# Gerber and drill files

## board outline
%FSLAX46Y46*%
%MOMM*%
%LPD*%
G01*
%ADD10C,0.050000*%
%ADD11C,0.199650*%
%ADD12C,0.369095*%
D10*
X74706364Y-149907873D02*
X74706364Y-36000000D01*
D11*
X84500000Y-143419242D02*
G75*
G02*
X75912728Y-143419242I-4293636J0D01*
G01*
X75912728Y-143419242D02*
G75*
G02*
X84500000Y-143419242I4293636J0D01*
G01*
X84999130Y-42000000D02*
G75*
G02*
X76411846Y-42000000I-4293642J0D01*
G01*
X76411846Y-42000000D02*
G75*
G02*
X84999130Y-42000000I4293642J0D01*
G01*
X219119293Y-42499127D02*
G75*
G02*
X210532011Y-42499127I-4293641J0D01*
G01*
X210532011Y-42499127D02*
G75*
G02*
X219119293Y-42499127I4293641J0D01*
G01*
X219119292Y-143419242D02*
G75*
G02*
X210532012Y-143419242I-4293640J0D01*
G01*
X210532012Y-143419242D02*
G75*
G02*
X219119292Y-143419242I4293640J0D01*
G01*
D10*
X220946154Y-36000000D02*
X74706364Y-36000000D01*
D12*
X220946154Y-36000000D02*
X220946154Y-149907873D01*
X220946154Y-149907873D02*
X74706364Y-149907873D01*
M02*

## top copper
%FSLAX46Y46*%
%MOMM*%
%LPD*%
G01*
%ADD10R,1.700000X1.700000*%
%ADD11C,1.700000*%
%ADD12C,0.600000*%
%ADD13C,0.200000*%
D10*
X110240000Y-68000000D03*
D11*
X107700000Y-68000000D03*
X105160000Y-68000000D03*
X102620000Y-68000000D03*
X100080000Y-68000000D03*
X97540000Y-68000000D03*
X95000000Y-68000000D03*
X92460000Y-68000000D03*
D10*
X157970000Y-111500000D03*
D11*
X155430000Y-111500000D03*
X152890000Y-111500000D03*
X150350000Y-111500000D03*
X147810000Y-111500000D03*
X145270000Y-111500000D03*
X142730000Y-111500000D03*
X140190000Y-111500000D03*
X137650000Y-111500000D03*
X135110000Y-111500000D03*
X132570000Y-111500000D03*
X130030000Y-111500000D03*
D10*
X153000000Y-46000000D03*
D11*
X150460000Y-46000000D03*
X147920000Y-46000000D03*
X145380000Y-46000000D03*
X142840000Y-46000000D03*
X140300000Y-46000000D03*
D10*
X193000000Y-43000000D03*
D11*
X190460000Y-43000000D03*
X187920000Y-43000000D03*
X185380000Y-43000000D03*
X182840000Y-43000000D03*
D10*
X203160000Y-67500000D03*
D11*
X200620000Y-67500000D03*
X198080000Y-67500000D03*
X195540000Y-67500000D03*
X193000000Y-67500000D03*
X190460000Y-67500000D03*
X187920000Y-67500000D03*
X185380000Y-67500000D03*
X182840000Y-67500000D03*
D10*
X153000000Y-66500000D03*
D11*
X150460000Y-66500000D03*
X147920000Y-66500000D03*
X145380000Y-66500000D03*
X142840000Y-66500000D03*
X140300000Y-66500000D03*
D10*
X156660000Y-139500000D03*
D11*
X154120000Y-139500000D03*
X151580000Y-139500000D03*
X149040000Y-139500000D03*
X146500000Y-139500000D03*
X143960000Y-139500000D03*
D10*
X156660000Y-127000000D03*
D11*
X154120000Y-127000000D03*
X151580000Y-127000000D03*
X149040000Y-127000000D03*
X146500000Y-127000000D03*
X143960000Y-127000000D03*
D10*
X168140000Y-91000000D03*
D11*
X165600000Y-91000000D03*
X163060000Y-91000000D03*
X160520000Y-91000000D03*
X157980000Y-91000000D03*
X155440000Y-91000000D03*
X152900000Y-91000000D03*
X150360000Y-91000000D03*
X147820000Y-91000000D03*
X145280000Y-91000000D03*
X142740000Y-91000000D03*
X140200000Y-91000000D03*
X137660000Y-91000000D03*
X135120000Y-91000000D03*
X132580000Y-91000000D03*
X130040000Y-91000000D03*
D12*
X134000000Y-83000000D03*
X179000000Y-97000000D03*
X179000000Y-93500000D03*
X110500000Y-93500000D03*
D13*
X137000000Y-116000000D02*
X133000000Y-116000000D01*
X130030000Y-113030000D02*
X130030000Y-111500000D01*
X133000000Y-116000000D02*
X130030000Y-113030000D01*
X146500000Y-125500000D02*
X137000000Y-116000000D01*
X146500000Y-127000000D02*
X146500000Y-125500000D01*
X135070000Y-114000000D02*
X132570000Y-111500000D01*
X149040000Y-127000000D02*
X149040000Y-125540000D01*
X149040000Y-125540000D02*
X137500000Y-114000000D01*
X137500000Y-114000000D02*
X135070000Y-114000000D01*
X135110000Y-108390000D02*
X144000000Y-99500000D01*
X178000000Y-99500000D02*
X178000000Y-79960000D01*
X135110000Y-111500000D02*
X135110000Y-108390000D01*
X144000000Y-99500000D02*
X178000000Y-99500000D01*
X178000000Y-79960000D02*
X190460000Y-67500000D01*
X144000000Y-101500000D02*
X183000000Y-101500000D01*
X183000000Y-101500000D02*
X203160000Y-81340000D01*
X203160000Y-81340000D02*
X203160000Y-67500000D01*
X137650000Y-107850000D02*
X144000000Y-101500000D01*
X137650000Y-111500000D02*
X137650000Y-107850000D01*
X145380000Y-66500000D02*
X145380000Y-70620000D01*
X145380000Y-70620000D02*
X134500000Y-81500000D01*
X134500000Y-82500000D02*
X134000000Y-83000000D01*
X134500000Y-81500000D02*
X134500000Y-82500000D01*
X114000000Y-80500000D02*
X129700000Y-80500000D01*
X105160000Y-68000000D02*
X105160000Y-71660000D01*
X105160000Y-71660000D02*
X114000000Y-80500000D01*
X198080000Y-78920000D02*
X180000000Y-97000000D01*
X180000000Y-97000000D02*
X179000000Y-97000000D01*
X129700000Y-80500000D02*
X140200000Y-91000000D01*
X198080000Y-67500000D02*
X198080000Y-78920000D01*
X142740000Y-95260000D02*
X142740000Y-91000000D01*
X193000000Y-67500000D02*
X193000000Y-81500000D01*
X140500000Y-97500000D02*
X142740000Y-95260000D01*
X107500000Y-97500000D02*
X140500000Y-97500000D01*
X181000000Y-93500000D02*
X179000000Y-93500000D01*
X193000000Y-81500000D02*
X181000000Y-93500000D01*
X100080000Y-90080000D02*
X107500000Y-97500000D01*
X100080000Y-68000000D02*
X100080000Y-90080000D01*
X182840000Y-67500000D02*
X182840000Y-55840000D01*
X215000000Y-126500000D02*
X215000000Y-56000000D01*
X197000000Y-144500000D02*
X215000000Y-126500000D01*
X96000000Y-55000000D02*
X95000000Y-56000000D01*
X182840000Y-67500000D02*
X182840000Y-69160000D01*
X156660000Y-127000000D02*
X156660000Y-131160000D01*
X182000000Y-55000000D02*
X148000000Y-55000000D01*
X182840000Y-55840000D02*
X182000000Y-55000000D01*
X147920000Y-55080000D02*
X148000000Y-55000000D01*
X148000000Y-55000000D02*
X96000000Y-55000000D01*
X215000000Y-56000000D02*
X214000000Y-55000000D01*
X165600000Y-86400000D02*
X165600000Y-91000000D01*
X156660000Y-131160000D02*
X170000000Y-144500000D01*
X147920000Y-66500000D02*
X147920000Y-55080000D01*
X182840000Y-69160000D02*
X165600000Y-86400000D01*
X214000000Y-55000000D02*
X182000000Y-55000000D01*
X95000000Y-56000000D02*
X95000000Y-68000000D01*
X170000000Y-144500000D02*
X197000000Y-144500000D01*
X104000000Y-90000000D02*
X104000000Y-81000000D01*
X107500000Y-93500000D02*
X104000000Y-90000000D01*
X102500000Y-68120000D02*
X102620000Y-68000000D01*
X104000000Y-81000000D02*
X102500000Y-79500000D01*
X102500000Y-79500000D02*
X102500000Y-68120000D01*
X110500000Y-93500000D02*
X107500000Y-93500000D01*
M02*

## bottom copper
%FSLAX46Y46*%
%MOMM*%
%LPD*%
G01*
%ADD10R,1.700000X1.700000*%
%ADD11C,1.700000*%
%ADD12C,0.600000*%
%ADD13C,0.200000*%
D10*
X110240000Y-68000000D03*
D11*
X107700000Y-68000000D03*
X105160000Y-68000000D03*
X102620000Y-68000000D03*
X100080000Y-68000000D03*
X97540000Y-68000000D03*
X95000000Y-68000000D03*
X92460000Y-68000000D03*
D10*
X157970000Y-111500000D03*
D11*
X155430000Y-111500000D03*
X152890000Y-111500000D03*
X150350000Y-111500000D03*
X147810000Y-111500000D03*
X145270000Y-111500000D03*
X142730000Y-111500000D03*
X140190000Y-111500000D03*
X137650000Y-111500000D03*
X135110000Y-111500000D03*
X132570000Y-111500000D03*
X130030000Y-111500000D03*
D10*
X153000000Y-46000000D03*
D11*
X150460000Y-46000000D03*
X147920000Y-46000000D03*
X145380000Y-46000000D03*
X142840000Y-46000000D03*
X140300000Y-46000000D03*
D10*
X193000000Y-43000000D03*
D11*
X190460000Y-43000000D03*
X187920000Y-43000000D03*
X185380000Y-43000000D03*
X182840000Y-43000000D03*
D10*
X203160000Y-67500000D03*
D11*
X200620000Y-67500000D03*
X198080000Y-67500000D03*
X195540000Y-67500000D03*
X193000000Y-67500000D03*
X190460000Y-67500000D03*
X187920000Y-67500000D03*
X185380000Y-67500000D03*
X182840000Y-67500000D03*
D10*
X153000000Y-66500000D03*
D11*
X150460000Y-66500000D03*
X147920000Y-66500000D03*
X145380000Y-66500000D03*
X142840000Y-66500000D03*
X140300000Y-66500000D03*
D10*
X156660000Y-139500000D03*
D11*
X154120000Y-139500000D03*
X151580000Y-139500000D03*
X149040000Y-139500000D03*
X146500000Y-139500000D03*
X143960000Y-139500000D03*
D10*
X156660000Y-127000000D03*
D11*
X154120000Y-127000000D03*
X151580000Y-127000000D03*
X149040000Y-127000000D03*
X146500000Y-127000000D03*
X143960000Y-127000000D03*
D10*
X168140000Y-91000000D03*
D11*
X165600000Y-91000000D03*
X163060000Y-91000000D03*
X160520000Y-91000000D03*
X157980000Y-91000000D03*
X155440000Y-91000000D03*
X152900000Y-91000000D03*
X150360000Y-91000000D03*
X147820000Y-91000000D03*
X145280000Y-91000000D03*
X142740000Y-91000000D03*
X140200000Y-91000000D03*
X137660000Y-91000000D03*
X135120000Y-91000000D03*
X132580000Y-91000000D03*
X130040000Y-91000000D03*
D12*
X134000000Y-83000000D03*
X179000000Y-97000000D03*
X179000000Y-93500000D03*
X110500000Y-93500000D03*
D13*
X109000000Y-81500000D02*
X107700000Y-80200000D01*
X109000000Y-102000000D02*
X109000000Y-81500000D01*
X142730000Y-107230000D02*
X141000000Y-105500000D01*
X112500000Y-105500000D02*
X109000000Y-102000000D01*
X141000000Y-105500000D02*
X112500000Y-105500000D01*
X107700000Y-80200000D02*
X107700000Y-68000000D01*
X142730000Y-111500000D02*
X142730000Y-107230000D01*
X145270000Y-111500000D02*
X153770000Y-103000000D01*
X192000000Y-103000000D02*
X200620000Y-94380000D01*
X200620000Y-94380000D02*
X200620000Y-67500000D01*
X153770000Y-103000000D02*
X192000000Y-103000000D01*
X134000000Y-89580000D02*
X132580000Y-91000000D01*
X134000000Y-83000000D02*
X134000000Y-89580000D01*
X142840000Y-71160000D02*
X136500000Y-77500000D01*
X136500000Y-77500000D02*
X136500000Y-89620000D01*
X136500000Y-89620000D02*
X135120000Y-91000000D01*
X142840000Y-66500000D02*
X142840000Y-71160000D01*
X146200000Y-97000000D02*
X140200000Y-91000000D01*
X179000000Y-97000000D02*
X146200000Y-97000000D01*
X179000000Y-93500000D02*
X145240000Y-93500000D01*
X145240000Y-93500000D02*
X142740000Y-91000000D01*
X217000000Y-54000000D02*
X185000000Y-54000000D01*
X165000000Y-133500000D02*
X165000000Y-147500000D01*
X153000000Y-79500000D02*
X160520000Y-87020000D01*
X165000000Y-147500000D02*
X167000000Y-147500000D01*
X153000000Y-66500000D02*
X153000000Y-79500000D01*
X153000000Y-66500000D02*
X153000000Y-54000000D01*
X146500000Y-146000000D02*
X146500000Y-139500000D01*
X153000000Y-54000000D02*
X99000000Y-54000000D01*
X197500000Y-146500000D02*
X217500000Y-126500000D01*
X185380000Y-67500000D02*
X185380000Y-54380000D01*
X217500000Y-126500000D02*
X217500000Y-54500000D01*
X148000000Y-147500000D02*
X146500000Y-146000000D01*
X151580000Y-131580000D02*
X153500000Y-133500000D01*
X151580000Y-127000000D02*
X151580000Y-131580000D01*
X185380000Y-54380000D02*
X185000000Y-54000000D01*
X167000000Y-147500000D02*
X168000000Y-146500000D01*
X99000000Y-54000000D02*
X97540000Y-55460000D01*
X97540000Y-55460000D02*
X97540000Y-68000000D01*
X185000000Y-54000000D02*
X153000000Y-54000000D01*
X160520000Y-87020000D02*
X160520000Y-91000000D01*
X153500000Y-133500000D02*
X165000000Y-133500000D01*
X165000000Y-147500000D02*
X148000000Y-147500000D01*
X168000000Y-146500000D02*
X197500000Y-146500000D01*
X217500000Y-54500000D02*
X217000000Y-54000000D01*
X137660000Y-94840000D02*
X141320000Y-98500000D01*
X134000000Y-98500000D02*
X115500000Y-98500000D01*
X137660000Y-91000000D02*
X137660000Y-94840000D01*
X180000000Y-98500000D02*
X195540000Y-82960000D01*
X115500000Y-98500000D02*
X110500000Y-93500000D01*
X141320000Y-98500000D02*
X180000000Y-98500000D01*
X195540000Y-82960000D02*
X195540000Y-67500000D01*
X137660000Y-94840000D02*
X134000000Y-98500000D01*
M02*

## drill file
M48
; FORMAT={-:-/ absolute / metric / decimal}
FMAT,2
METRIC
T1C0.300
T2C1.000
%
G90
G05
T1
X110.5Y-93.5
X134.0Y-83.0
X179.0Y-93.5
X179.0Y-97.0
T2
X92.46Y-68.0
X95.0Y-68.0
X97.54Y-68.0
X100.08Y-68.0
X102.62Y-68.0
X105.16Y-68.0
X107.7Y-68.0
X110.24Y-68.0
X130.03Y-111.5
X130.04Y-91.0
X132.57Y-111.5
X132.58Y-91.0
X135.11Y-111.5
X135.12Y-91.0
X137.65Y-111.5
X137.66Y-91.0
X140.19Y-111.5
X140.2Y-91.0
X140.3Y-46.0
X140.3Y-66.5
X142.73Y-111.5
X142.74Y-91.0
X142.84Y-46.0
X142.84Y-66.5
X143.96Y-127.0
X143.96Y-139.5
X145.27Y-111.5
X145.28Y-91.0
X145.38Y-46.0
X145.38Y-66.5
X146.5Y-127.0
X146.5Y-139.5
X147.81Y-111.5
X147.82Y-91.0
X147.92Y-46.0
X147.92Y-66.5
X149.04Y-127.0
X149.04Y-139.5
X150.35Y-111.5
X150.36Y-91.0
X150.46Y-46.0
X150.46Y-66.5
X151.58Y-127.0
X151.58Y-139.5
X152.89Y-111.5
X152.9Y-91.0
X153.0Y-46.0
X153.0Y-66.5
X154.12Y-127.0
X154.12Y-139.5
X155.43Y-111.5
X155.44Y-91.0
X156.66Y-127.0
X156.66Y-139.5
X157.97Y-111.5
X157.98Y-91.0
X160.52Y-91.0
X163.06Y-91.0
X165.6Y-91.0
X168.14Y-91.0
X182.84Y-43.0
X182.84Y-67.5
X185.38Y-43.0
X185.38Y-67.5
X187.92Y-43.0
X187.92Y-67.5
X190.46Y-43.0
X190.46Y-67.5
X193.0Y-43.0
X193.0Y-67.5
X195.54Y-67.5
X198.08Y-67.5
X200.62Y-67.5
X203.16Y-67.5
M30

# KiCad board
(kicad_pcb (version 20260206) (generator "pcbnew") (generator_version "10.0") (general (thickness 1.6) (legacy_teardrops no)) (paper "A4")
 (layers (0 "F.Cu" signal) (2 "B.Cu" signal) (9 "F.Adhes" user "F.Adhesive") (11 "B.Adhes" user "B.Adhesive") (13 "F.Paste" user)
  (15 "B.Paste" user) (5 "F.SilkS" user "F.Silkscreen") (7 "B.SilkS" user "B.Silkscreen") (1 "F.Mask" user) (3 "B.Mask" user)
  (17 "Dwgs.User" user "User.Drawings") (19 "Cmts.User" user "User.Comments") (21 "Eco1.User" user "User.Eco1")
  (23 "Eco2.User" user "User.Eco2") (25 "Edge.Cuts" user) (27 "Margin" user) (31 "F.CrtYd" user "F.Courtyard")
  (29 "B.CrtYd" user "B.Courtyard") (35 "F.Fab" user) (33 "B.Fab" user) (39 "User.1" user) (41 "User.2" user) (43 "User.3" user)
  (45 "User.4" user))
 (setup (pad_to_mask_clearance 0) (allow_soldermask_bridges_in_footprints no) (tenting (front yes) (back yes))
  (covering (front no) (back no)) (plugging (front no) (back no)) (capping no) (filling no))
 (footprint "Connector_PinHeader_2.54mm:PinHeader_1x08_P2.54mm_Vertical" (layer "F.Cu") (at 110.24 68 -90)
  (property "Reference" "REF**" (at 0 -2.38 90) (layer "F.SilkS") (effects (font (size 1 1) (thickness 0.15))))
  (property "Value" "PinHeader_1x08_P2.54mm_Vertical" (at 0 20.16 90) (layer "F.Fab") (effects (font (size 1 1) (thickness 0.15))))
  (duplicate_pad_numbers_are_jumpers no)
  (pad "1" thru_hole rect (at 0 0 270) (size 1.7 1.7) (drill 1) (layers "*.Cu" "*.Mask") (remove_unused_layers no))
  (pad "2" thru_hole circle (at 0 2.54 270) (size 1.7 1.7) (drill 1) (layers "*.Cu" "*.Mask") (remove_unused_layers no) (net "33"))
  (pad "3" thru_hole circle (at 0 5.08 270) (size 1.7 1.7) (drill 1) (layers "*.Cu" "*.Mask") (remove_unused_layers no) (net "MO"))
  (pad "4" thru_hole circle (at 0 7.62 270) (size 1.7 1.7) (drill 1) (layers "*.Cu" "*.Mask") (remove_unused_layers no) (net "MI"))
  (pad "5" thru_hole circle (at 0 10.16 270) (size 1.7 1.7) (drill 1) (layers "*.Cu" "*.Mask") (remove_unused_layers no) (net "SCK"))
  (pad "6" thru_hole circle (at 0 12.7 270) (size 1.7 1.7) (drill 1) (layers "*.Cu" "*.Mask") (remove_unused_layers no) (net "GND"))
  (pad "7" thru_hole circle (at 0 15.24 270) (size 1.7 1.7) (drill 1) (layers "*.Cu" "*.Mask") (remove_unused_layers no) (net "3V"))
  (pad "8" thru_hole circle (at 0 17.78 270) (size 1.7 1.7) (drill 1) (layers "*.Cu" "*.Mask") (remove_unused_layers no)))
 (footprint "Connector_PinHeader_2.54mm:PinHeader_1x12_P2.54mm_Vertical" (layer "F.Cu") (at 157.97 111.5 -90)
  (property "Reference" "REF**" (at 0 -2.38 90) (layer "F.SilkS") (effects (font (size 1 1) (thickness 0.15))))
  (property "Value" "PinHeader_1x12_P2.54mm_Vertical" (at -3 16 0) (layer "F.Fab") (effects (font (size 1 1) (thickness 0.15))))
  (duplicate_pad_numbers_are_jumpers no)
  (pad "1" thru_hole rect (at 0 0 270) (size 1.7 1.7) (drill 1) (layers "*.Cu" "*.Mask") (remove_unused_layers no))
  (pad "2" thru_hole circle (at 0 2.54 270) (size 1.7 1.7) (drill 1) (layers "*.Cu" "*.Mask") (remove_unused_layers no))
  (pad "3" thru_hole circle (at 0 5.08 270) (size 1.7 1.7) (drill 1) (layers "*.Cu" "*.Mask") (remove_unused_layers no))
  (pad "4" thru_hole circle (at 0 7.62 270) (size 1.7 1.7) (drill 1) (layers "*.Cu" "*.Mask") (remove_unused_layers no))
  (pad "5" thru_hole circle (at 0 10.16 270) (size 1.7 1.7) (drill 1) (layers "*.Cu" "*.Mask") (remove_unused_layers no))
  (pad "6" thru_hole circle (at 0 12.7 270) (size 1.7 1.7) (drill 1) (layers "*.Cu" "*.Mask") (remove_unused_layers no) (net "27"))
  (pad "7" thru_hole circle (at 0 15.24 270) (size 1.7 1.7) (drill 1) (layers "*.Cu" "*.Mask") (remove_unused_layers no) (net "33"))
  (pad "8" thru_hole circle (at 0 17.78 270) (size 1.7 1.7) (drill 1) (layers "*.Cu" "*.Mask") (remove_unused_layers no))
  (pad "9" thru_hole circle (at 0 20.32 270) (size 1.7 1.7) (drill 1) (layers "*.Cu" "*.Mask") (remove_unused_layers no) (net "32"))
  (pad "10" thru_hole circle (at 0 22.86 270) (size 1.7 1.7) (drill 1) (layers "*.Cu" "*.Mask") (remove_unused_layers no) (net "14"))
  (pad "11" thru_hole circle (at 0 25.4 270) (size 1.7 1.7) (drill 1) (layers "*.Cu" "*.Mask") (remove_unused_layers no) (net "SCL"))
  (pad "12" thru_hole circle (at 0 27.94 270) (size 1.7 1.7) (drill 1) (layers "*.Cu" "*.Mask") (remove_unused_layers no) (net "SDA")))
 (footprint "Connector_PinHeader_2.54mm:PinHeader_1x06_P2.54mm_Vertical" (layer "F.Cu") (at 153 46 -90)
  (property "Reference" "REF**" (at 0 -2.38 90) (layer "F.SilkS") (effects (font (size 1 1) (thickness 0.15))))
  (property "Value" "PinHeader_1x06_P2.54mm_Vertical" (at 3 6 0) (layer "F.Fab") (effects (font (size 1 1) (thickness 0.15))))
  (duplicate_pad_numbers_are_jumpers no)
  (pad "1" thru_hole rect (at 0 0 270) (size 1.7 1.7) (drill 1) (layers "*.Cu" "*.Mask") (remove_unused_layers no))
  (pad "2" thru_hole circle (at 0 2.54 270) (size 1.7 1.7) (drill 1) (layers "*.Cu" "*.Mask") (remove_unused_layers no))
  (pad "3" thru_hole circle (at 0 5.08 270) (size 1.7 1.7) (drill 1) (layers "*.Cu" "*.Mask") (remove_unused_layers no))
  (pad "4" thru_hole circle (at 0 7.62 270) (size 1.7 1.7) (drill 1) (layers "*.Cu" "*.Mask") (remove_unused_layers no))
  (pad "5" thru_hole circle (at 0 10.16 270) (size 1.7 1.7) (drill 1) (layers "*.Cu" "*.Mask") (remove_unused_layers no))
  (pad "6" thru_hole circle (at 0 12.7 270) (size 1.7 1.7) (drill 1) (layers "*.Cu" "*.Mask") (remove_unused_layers no)))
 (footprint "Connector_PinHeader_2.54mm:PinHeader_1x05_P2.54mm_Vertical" (layer "F.Cu") (at 193 43 -90)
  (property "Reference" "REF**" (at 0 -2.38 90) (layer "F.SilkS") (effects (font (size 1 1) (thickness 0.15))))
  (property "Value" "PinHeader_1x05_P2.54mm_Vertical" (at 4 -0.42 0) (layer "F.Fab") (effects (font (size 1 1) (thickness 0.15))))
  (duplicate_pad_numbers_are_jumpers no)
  (pad "1" thru_hole rect (at 0 0 270) (size 1.7 1.7) (drill 1) (layers "*.Cu" "*.Mask") (remove_unused_layers no))
  (pad "2" thru_hole circle (at 0 2.54 270) (size 1.7 1.7) (drill 1) (layers "*.Cu" "*.Mask") (remove_unused_layers no))
  (pad "3" thru_hole circle (at 0 5.08 270) (size 1.7 1.7) (drill 1) (layers "*.Cu" "*.Mask") (remove_unused_layers no))
  (pad "4" thru_hole circle (at 0 7.62 270) (size 1.7 1.7) (drill 1) (layers "*.Cu" "*.Mask") (remove_unused_layers no))
  (pad "5" thru_hole circle (at 0 10.16 270) (size 1.7 1.7) (drill 1) (layers "*.Cu" "*.Mask") (remove_unused_layers no)))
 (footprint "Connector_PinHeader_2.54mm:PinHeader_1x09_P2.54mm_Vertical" (layer "F.Cu") (at 203.16 67.5 -90)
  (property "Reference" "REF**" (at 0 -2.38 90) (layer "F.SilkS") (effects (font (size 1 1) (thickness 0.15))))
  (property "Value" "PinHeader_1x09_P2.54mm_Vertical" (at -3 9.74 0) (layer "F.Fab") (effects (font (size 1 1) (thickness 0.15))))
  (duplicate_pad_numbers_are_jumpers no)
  (pad "1" thru_hole rect (at 0 0 270) (size 1.7 1.7) (drill 1) (layers "*.Cu" "*.Mask") (remove_unused_layers no) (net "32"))
  (pad "2" thru_hole circle (at 0 2.54 270) (size 1.7 1.7) (drill 1) (layers "*.Cu" "*.Mask") (remove_unused_layers no) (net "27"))
  (pad "3" thru_hole circle (at 0 5.08 270) (size 1.7 1.7) (drill 1) (layers "*.Cu" "*.Mask") (remove_unused_layers no) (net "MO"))
  (pad "4" thru_hole circle (at 0 7.62 270) (size 1.7 1.7) (drill 1) (layers "*.Cu" "*.Mask") (remove_unused_layers no) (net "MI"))
  (pad "5" thru_hole circle (at 0 10.16 270) (size 1.7 1.7) (drill 1) (layers "*.Cu" "*.Mask") (remove_unused_layers no) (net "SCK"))
  (pad "6" thru_hole circle (at 0 12.7 270) (size 1.7 1.7) (drill 1) (layers "*.Cu" "*.Mask") (remove_unused_layers no) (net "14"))
  (pad "7" thru_hole circle (at 0 15.24 270) (size 1.7 1.7) (drill 1) (layers "*.Cu" "*.Mask") (remove_unused_layers no))
  (pad "8" thru_hole circle (at 0 17.78 270) (size 1.7 1.7) (drill 1) (layers "*.Cu" "*.Mask") (remove_unused_layers no) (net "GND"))
  (pad "9" thru_hole circle (at 0 20.32 270) (size 1.7 1.7) (drill 1) (layers "*.Cu" "*.Mask") (remove_unused_layers no) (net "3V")))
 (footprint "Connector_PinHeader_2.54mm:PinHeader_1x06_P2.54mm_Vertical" (layer "F.Cu") (at 153 66.5 -90)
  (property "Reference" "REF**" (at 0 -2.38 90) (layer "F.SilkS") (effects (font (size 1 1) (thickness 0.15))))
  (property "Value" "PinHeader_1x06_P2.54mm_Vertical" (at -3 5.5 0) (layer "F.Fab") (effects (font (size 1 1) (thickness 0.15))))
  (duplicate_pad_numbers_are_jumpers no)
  (pad "1" thru_hole rect (at 0 0 270) (size 1.7 1.7) (drill 1) (layers "*.Cu" "*.Mask") (remove_unused_layers no) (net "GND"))
  (pad "2" thru_hole circle (at 0 2.54 270) (size 1.7 1.7) (drill 1) (layers "*.Cu" "*.Mask") (remove_unused_layers no))
  (pad "3" thru_hole circle (at 0 5.08 270) (size 1.7 1.7) (drill 1) (layers "*.Cu" "*.Mask") (remove_unused_layers no) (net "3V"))
  (pad "4" thru_hole circle (at 0 7.62 270) (size 1.7 1.7) (drill 1) (layers "*.Cu" "*.Mask") (remove_unused_layers no) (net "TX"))
  (pad "5" thru_hole circle (at 0 10.16 270) (size 1.7 1.7) (drill 1) (layers "*.Cu" "*.Mask") (remove_unused_layers no) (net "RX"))
  (pad "6" thru_hole circle (at 0 12.7 270) (size 1.7 1.7) (drill 1) (layers "*.Cu" "*.Mask") (remove_unused_layers no)))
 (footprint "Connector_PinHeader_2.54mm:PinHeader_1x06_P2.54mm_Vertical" (layer "F.Cu") (at 156.66 139.5 -90)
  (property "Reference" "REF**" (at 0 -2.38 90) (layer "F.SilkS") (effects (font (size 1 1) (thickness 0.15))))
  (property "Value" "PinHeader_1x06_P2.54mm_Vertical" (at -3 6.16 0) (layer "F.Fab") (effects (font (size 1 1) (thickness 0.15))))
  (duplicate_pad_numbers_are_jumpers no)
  (pad "1" thru_hole rect (at 0 0 270) (size 1.7 1.7) (drill 1) (layers "*.Cu" "*.Mask") (remove_unused_layers no))
  (pad "2" thru_hole circle (at 0 2.54 270) (size 1.7 1.7) (drill 1) (layers "*.Cu" "*.Mask") (remove_unused_layers no))
  (pad "3" thru_hole circle (at 0 5.08 270) (size 1.7 1.7) (drill 1) (layers "*.Cu" "*.Mask") (remove_unused_layers no))
  (pad "4" thru_hole circle (at 0 7.62 270) (size 1.7 1.7) (drill 1) (layers "*.Cu" "*.Mask") (remove_unused_layers no))
  (pad "5" thru_hole circle (at 0 10.16 270) (size 1.7 1.7) (drill 1) (layers "*.Cu" "*.Mask") (remove_unused_layers no) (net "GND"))
  (pad "6" thru_hole circle (at 0 12.7 270) (size 1.7 1.7) (drill 1) (layers "*.Cu" "*.Mask") (remove_unused_layers no)))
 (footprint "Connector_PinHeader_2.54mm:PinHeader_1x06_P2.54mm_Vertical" (layer "F.Cu") (at 156.66 127 -90)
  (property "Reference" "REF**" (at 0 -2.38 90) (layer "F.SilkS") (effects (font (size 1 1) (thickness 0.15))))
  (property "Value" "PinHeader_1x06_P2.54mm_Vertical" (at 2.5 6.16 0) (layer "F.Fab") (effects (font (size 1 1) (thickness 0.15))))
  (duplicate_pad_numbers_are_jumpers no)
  (pad "1" thru_hole rect (at 0 0 270) (size 1.7 1.7) (drill 1) (layers "*.Cu" "*.Mask") (remove_unused_layers no) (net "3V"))
  (pad "2" thru_hole circle (at 0 2.54 270) (size 1.7 1.7) (drill 1) (layers "*.Cu" "*.Mask") (remove_unused_layers no))
  (pad "3" thru_hole circle (at 0 5.08 270) (size 1.7 1.7) (drill 1) (layers "*.Cu" "*.Mask") (remove_unused_layers no) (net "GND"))
  (pad "4" thru_hole circle (at 0 7.62 270) (size 1.7 1.7) (drill 1) (layers "*.Cu" "*.Mask") (remove_unused_layers no) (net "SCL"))
  (pad "5" thru_hole circle (at 0 10.16 270) (size 1.7 1.7) (drill 1) (layers "*.Cu" "*.Mask") (remove_unused_layers no) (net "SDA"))
  (pad "6" thru_hole circle (at 0 12.7 270) (size 1.7 1.7) (drill 1) (layers "*.Cu" "*.Mask") (remove_unused_layers no)))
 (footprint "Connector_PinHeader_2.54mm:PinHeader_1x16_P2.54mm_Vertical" (layer "F.Cu") (at 168.14 91 -90)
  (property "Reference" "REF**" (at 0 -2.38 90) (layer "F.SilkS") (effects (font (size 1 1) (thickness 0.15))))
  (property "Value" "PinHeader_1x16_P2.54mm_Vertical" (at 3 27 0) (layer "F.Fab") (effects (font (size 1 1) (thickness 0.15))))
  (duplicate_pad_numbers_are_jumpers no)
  (pad "1" thru_hole rect (at 0 0 270) (size 1.7 1.7) (drill 1) (layers "*.Cu" "*.Mask") (remove_unused_layers no))
  (pad "2" thru_hole circle (at 0 2.54 270) (size 1.7 1.7) (drill 1) (layers "*.Cu" "*.Mask") (remove_unused_layers no) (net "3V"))
  (pad "3" thru_hole circle (at 0 5.08 270) (size 1.7 1.7) (drill 1) (layers "*.Cu" "*.Mask") (remove_unused_layers no))
  (pad "4" thru_hole circle (at 0 7.62 270) (size 1.7 1.7) (drill 1) (layers "*.Cu" "*.Mask") (remove_unused_layers no) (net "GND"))
  (pad "5" thru_hole circle (at 0 10.16 270) (size 1.7 1.7) (drill 1) (layers "*.Cu" "*.Mask") (remove_unused_layers no))
  (pad "6" thru_hole circle (at 0 12.7 270) (size 1.7 1.7) (drill 1) (layers "*.Cu" "*.Mask") (remove_unused_layers no))
  (pad "7" thru_hole circle (at 0 15.24 270) (size 1.7 1.7) (drill 1) (layers "*.Cu" "*.Mask") (remove_unused_layers no))
  (pad "8" thru_hole circle (at 0 17.78 270) (size 1.7 1.7) (drill 1) (layers "*.Cu" "*.Mask") (remove_unused_layers no))
  (pad "9" thru_hole circle (at 0 20.32 270) (size 1.7 1.7) (drill 1) (layers "*.Cu" "*.Mask") (remove_unused_layers no))
  (pad "10" thru_hole circle (at 0 22.86 270) (size 1.7 1.7) (drill 1) (layers "*.Cu" "*.Mask") (remove_unused_layers no))
  (pad "11" thru_hole circle (at 0 25.4 270) (size 1.7 1.7) (drill 1) (layers "*.Cu" "*.Mask") (remove_unused_layers no) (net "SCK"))
  (pad "12" thru_hole circle (at 0 27.94 270) (size 1.7 1.7) (drill 1) (layers "*.Cu" "*.Mask") (remove_unused_layers no) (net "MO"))
  (pad "13" thru_hole circle (at 0 30.48 270) (size 1.7 1.7) (drill 1) (layers "*.Cu" "*.Mask") (remove_unused_layers no) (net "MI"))
  (pad "14" thru_hole circle (at 0 33.02 270) (size 1.7 1.7) (drill 1) (layers "*.Cu" "*.Mask") (remove_unused_layers no) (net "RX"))
  (pad "15" thru_hole circle (at 0 35.56 270) (size 1.7 1.7) (drill 1) (layers "*.Cu" "*.Mask") (remove_unused_layers no) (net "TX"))
  (pad "16" thru_hole circle (at 0 38.1 270) (size 1.7 1.7) (drill 1) (layers "*.Cu" "*.Mask") (remove_unused_layers no)))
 (gr_line (start 74.706364 149.907873) (end 74.706364 36) (stroke (width 0.05) (type default)) (layer "Edge.Cuts"))
 (gr_circle (center 80.206364 143.419242) (end 83.70024 145.914866) (stroke (width 0.19965) (type default)) (fill no) (layer "Edge.Cuts"))
 (gr_circle (center 80.705488 42) (end 84.199367 44.495631) (stroke (width 0.19965) (type default)) (fill no) (layer "Edge.Cuts"))
 (gr_circle (center 214.825652 42.499127) (end 218.31953 44.994757) (stroke (width 0.19965) (type default)) (fill no) (layer "Edge.Cuts"))
 (gr_circle (center 214.825652 143.419242) (end 218.31953 140.923613) (stroke (width 0.19965) (type default)) (fill no) (layer "Edge.Cuts"))
 (gr_line (start 220.946154 36) (end 74.706364 36) (stroke (width 0.05) (type default)) (layer "Edge.Cuts"))
 (gr_line (start 220.946154 36) (end 220.946154 149.907873) (stroke (width 0.369095) (type default)) (layer "Edge.Cuts"))
 (gr_line (start 220.946154 149.907873) (end 74.706364 149.907873) (stroke (width 0.369095) (type default)) (layer "Edge.Cuts"))
 (segment (start 137 116) (end 133 116) (width 0.2) (layer "F.Cu") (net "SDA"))
 (segment (start 130.03 113.03) (end 130.03 111.5) (width 0.2) (layer "F.Cu") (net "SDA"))
 (segment (start 133 116) (end 130.03 113.03) (width 0.2) (layer "F.Cu") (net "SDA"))
 (segment (start 146.5 125.5) (end 137 116) (width 0.2) (layer "F.Cu") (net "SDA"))
 (segment (start 146.5 127) (end 146.5 125.5) (width 0.2) (layer "F.Cu") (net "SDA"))
 (segment (start 135.07 114) (end 132.57 111.5) (width 0.2) (layer "F.Cu") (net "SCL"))
 (segment (start 149.04 127) (end 149.04 125.54) (width 0.2) (layer "F.Cu") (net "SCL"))
 (segment (start 149.04 125.54) (end 137.5 114) (width 0.2) (layer "F.Cu") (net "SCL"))
 (segment (start 137.5 114) (end 135.07 114) (width 0.2) (layer "F.Cu") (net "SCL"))
 (segment (start 135.11 108.39) (end 144 99.5) (width 0.2) (layer "F.Cu") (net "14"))
 (segment (start 178 99.5) (end 178 79.96) (width 0.2) (layer "F.Cu") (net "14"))
 (segment (start 135.11 111.5) (end 135.11 108.39) (width 0.2) (layer "F.Cu") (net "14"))
 (segment (start 144 99.5) (end 178 99.5) (width 0.2) (layer "F.Cu") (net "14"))
 (segment (start 178 79.96) (end 190.46 67.5) (width 0.2) (layer "F.Cu") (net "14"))
 (segment (start 144 101.5) (end 183 101.5) (width 0.2) (layer "F.Cu") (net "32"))
 (segment (start 183 101.5) (end 203.16 81.34) (width 0.2) (layer "F.Cu") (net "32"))
 (segment (start 203.16 81.34) (end 203.16 67.5) (width 0.2) (layer "F.Cu") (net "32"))
 (segment (start 137.65 107.85) (end 144 101.5) (width 0.2) (layer "F.Cu") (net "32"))
 (segment (start 137.65 111.5) (end 137.65 107.85) (width 0.2) (layer "F.Cu") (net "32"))
 (segment (start 109 81.5) (end 107.7 80.2) (width 0.2) (layer "B.Cu") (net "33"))
 (segment (start 109 102) (end 109 81.5) (width 0.2) (layer "B.Cu") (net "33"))
 (segment (start 142.73 107.23) (end 141 105.5) (width 0.2) (layer "B.Cu") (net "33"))
 (segment (start 112.5 105.5) (end 109 102) (width 0.2) (layer "B.Cu") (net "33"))
 (segment (start 141 105.5) (end 112.5 105.5) (width 0.2) (layer "B.Cu") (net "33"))
 (segment (start 107.7 80.2) (end 107.7 68) (width 0.2) (layer "B.Cu") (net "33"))
 (segment (start 142.73 111.5) (end 142.73 107.23) (width 0.2) (layer "B.Cu") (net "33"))
 (segment (start 145.27 111.5) (end 153.77 103) (width 0.2) (layer "B.Cu") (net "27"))
 (segment (start 192 103) (end 200.62 94.38) (width 0.2) (layer "B.Cu") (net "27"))
 (segment (start 200.62 94.38) (end 200.62 67.5) (width 0.2) (layer "B.Cu") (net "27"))
 (segment (start 153.77 103) (end 192 103) (width 0.2) (layer "B.Cu") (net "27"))
 (segment (start 145.38 66.5) (end 145.38 70.62) (width 0.2) (layer "F.Cu") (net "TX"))
 (segment (start 145.38 70.62) (end 134.5 81.5) (width 0.2) (layer "F.Cu") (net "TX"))
 (segment (start 134.5 82.5) (end 134 83) (width 0.2) (layer "F.Cu") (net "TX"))
 (segment (start 134.5 81.5) (end 134.5 82.5) (width 0.2) (layer "F.Cu") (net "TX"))
 (via (at 134 83) (size 0.6) (drill 0.3) (layers "F.Cu" "B.Cu") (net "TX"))
 (segment (start 134 89.58) (end 132.58 91) (width 0.2) (layer "B.Cu") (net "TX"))
 (segment (start 134 83) (end 134 89.58) (width 0.2) (layer "B.Cu") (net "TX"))
 (segment (start 142.84 71.16) (end 136.5 77.5) (width 0.2) (layer "B.Cu") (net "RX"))
 (segment (start 136.5 77.5) (end 136.5 89.62) (width 0.2) (layer "B.Cu") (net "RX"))
 (segment (start 136.5 89.62) (end 135.12 91) (width 0.2) (layer "B.Cu") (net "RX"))
 (segment (start 142.84 66.5) (end 142.84 71.16) (width 0.2) (layer "B.Cu") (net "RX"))
 (segment (start 114 80.5) (end 129.7 80.5) (width 0.2) (layer "F.Cu") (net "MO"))
 (segment (start 105.16 68) (end 105.16 71.66) (width 0.2) (layer "F.Cu") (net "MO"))
 (segment (start 105.16 71.66) (end 114 80.5) (width 0.2) (layer "F.Cu") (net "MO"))
 (segment (start 198.08 78.92) (end 180 97) (width 0.2) (layer "F.Cu") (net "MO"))
 (segment (start 180 97) (end 179 97) (width 0.2) (layer "F.Cu") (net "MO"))
 (segment (start 129.7 80.5) (end 140.2 91) (width 0.2) (layer "F.Cu") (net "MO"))
 (segment (start 198.08 67.5) (end 198.08 78.92) (width 0.2) (layer "F.Cu") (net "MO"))
 (via (at 179 97) (size 0.6) (drill 0.3) (layers "F.Cu" "B.Cu") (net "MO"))
 (segment (start 146.2 97) (end 140.2 91) (width 0.2) (layer "B.Cu") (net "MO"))
 (segment (start 179 97) (end 146.2 97) (width 0.2) (layer "B.Cu") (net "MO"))
 (segment (start 142.74 95.26) (end 142.74 91) (width 0.2) (layer "F.Cu") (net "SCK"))
 (segment (start 193 67.5) (end 193 81.5) (width 0.2) (layer "F.Cu") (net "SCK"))
 (segment (start 140.5 97.5) (end 142.74 95.26) (width 0.2) (layer "F.Cu") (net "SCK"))
 (segment (start 107.5 97.5) (end 140.5 97.5) (width 0.2) (layer "F.Cu") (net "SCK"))
 (segment (start 181 93.5) (end 179 93.5) (width 0.2) (layer "F.Cu") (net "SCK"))
 (segment (start 193 81.5) (end 181 93.5) (width 0.2) (layer "F.Cu") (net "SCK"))
 (segment (start 100.08 90.08) (end 107.5 97.5) (width 0.2) (layer "F.Cu") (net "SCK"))
 (segment (start 100.08 68) (end 100.08 90.08) (width 0.2) (layer "F.Cu") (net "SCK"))
 (via (at 179 93.5) (size 0.6) (drill 0.3) (layers "F.Cu" "B.Cu") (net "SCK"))
 (segment (start 179 93.5) (end 145.24 93.5) (width 0.2) (layer "B.Cu") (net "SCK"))
 (segment (start 145.24 93.5) (end 142.74 91) (width 0.2) (layer "B.Cu") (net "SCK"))
 (segment (start 182.84 67.5) (end 182.84 55.84) (width 0.2) (layer "F.Cu") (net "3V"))
 (segment (start 215 126.5) (end 215 56) (width 0.2) (layer "F.Cu") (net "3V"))
 (segment (start 197 144.5) (end 215 126.5) (width 0.2) (layer "F.Cu") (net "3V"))
 (segment (start 96 55) (end 95 56) (width 0.2) (layer "F.Cu") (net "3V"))
 (segment (start 182.84 67.5) (end 182.84 69.16) (width 0.2) (layer "F.Cu") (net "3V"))
 (segment (start 156.66 127) (end 156.66 131.16) (width 0.2) (layer "F.Cu") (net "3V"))
 (segment (start 182 55) (end 148 55) (width 0.2) (layer "F.Cu") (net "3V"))
 (segment (start 182.84 55.84) (end 182 55) (width 0.2) (layer "F.Cu") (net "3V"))
 (segment (start 147.92 55.08) (end 148 55) (width 0.2) (layer "F.Cu") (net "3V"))
 (segment (start 148 55) (end 96 55) (width 0.2) (layer "F.Cu") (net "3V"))
 (segment (start 215 56) (end 214 55) (width 0.2) (layer "F.Cu") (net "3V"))
 (segment (start 165.6 86.4) (end 165.6 91) (width 0.2) (layer "F.Cu") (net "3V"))
 (segment (start 156.66 131.16) (end 170 144.5) (width 0.2) (layer "F.Cu") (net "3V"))
 (segment (start 147.92 66.5) (end 147.92 55.08) (width 0.2) (layer "F.Cu") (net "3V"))
 (segment (start 182.84 69.16) (end 165.6 86.4) (width 0.2) (layer "F.Cu") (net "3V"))
 (segment (start 214 55) (end 182 55) (width 0.2) (layer "F.Cu") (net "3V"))
 (segment (start 95 56) (end 95 68) (width 0.2) (layer "F.Cu") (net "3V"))
 (segment (start 170 144.5) (end 197 144.5) (width 0.2) (layer "F.Cu") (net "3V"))
 (segment (start 217 54) (end 185 54) (width 0.2) (layer "B.Cu") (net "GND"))
 (segment (start 165 133.5) (end 165 147.5) (width 0.2) (layer "B.Cu") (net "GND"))
 (segment (start 153 79.5) (end 160.52 87.02) (width 0.2) (layer "B.Cu") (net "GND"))
 (segment (start 165 147.5) (end 167 147.5) (width 0.2) (layer "B.Cu") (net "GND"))
 (segment (start 153 66.5) (end 153 79.5) (width 0.2) (layer "B.Cu") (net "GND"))
 (segment (start 153 66.5) (end 153 54) (width 0.2) (layer "B.Cu") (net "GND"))
 (segment (start 146.5 146) (end 146.5 139.5) (width 0.2) (layer "B.Cu") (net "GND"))
 (segment (start 153 54) (end 99 54) (width 0.2) (layer "B.Cu") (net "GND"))
 (segment (start 197.5 146.5) (end 217.5 126.5) (width 0.2) (layer "B.Cu") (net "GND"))
 (segment (start 185.38 67.5) (end 185.38 54.38) (width 0.2) (layer "B.Cu") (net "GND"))
 (segment (start 217.5 126.5) (end 217.5 54.5) (width 0.2) (layer "B.Cu") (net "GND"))
 (segment (start 148 147.5) (end 146.5 146) (width 0.2) (layer "B.Cu") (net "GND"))
 (segment (start 151.58 131.58) (end 153.5 133.5) (width 0.2) (layer "B.Cu") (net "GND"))
 (segment (start 151.58 127) (end 151.58 131.58) (width 0.2) (layer "B.Cu") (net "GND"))
 (segment (start 185.38 54.38) (end 185 54) (width 0.2) (layer "B.Cu") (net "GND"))
 (segment (start 167 147.5) (end 168 146.5) (width 0.2) (layer "B.Cu") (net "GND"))
 (segment (start 99 54) (end 97.54 55.46) (width 0.2) (layer "B.Cu") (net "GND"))
 (segment (start 97.54 55.46) (end 97.54 68) (width 0.2) (layer "B.Cu") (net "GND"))
 (segment (start 185 54) (end 153 54) (width 0.2) (layer "B.Cu") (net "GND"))
 (segment (start 160.52 87.02) (end 160.52 91) (width 0.2) (layer "B.Cu") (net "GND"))
 (segment (start 153.5 133.5) (end 165 133.5) (width 0.2) (layer "B.Cu") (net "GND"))
 (segment (start 165 147.5) (end 148 147.5) (width 0.2) (layer "B.Cu") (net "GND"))
 (segment (start 168 146.5) (end 197.5 146.5) (width 0.2) (layer "B.Cu") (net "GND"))
 (segment (start 217.5 54.5) (end 217 54) (width 0.2) (layer "B.Cu") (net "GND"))
 (segment (start 104 90) (end 104 81) (width 0.2) (layer "F.Cu") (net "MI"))
 (segment (start 107.5 93.5) (end 104 90) (width 0.2) (layer "F.Cu") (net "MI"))
 (segment (start 102.5 68.12) (end 102.62 68) (width 0.2) (layer "F.Cu") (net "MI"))
 (segment (start 104 81) (end 102.5 79.5) (width 0.2) (layer "F.Cu") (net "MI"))
 (segment (start 102.5 79.5) (end 102.5 68.12) (width 0.2) (layer "F.Cu") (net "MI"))
 (segment (start 110.5 93.5) (end 107.5 93.5) (width 0.2) (layer "F.Cu") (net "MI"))
 (via (at 110.5 93.5) (size 0.6) (drill 0.3) (layers "F.Cu" "B.Cu") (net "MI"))
 (segment (start 137.66 94.84) (end 141.32 98.5) (width 0.2) (layer "B.Cu") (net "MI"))
 (segment (start 134 98.5) (end 115.5 98.5) (width 0.2) (layer "B.Cu") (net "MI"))
 (segment (start 137.66 91) (end 137.66 94.84) (width 0.2) (layer "B.Cu") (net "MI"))
 (segment (start 180 98.5) (end 195.54 82.96) (width 0.2) (layer "B.Cu") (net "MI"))
 (segment (start 115.5 98.5) (end 110.5 93.5) (width 0.2) (layer "B.Cu") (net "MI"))
 (segment (start 141.32 98.5) (end 180 98.5) (width 0.2) (layer "B.Cu") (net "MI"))
 (segment (start 195.54 82.96) (end 195.54 67.5) (width 0.2) (layer "B.Cu") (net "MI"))
 (segment (start 137.66 94.84) (end 134 98.5) (width 0.2) (layer "B.Cu") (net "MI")))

